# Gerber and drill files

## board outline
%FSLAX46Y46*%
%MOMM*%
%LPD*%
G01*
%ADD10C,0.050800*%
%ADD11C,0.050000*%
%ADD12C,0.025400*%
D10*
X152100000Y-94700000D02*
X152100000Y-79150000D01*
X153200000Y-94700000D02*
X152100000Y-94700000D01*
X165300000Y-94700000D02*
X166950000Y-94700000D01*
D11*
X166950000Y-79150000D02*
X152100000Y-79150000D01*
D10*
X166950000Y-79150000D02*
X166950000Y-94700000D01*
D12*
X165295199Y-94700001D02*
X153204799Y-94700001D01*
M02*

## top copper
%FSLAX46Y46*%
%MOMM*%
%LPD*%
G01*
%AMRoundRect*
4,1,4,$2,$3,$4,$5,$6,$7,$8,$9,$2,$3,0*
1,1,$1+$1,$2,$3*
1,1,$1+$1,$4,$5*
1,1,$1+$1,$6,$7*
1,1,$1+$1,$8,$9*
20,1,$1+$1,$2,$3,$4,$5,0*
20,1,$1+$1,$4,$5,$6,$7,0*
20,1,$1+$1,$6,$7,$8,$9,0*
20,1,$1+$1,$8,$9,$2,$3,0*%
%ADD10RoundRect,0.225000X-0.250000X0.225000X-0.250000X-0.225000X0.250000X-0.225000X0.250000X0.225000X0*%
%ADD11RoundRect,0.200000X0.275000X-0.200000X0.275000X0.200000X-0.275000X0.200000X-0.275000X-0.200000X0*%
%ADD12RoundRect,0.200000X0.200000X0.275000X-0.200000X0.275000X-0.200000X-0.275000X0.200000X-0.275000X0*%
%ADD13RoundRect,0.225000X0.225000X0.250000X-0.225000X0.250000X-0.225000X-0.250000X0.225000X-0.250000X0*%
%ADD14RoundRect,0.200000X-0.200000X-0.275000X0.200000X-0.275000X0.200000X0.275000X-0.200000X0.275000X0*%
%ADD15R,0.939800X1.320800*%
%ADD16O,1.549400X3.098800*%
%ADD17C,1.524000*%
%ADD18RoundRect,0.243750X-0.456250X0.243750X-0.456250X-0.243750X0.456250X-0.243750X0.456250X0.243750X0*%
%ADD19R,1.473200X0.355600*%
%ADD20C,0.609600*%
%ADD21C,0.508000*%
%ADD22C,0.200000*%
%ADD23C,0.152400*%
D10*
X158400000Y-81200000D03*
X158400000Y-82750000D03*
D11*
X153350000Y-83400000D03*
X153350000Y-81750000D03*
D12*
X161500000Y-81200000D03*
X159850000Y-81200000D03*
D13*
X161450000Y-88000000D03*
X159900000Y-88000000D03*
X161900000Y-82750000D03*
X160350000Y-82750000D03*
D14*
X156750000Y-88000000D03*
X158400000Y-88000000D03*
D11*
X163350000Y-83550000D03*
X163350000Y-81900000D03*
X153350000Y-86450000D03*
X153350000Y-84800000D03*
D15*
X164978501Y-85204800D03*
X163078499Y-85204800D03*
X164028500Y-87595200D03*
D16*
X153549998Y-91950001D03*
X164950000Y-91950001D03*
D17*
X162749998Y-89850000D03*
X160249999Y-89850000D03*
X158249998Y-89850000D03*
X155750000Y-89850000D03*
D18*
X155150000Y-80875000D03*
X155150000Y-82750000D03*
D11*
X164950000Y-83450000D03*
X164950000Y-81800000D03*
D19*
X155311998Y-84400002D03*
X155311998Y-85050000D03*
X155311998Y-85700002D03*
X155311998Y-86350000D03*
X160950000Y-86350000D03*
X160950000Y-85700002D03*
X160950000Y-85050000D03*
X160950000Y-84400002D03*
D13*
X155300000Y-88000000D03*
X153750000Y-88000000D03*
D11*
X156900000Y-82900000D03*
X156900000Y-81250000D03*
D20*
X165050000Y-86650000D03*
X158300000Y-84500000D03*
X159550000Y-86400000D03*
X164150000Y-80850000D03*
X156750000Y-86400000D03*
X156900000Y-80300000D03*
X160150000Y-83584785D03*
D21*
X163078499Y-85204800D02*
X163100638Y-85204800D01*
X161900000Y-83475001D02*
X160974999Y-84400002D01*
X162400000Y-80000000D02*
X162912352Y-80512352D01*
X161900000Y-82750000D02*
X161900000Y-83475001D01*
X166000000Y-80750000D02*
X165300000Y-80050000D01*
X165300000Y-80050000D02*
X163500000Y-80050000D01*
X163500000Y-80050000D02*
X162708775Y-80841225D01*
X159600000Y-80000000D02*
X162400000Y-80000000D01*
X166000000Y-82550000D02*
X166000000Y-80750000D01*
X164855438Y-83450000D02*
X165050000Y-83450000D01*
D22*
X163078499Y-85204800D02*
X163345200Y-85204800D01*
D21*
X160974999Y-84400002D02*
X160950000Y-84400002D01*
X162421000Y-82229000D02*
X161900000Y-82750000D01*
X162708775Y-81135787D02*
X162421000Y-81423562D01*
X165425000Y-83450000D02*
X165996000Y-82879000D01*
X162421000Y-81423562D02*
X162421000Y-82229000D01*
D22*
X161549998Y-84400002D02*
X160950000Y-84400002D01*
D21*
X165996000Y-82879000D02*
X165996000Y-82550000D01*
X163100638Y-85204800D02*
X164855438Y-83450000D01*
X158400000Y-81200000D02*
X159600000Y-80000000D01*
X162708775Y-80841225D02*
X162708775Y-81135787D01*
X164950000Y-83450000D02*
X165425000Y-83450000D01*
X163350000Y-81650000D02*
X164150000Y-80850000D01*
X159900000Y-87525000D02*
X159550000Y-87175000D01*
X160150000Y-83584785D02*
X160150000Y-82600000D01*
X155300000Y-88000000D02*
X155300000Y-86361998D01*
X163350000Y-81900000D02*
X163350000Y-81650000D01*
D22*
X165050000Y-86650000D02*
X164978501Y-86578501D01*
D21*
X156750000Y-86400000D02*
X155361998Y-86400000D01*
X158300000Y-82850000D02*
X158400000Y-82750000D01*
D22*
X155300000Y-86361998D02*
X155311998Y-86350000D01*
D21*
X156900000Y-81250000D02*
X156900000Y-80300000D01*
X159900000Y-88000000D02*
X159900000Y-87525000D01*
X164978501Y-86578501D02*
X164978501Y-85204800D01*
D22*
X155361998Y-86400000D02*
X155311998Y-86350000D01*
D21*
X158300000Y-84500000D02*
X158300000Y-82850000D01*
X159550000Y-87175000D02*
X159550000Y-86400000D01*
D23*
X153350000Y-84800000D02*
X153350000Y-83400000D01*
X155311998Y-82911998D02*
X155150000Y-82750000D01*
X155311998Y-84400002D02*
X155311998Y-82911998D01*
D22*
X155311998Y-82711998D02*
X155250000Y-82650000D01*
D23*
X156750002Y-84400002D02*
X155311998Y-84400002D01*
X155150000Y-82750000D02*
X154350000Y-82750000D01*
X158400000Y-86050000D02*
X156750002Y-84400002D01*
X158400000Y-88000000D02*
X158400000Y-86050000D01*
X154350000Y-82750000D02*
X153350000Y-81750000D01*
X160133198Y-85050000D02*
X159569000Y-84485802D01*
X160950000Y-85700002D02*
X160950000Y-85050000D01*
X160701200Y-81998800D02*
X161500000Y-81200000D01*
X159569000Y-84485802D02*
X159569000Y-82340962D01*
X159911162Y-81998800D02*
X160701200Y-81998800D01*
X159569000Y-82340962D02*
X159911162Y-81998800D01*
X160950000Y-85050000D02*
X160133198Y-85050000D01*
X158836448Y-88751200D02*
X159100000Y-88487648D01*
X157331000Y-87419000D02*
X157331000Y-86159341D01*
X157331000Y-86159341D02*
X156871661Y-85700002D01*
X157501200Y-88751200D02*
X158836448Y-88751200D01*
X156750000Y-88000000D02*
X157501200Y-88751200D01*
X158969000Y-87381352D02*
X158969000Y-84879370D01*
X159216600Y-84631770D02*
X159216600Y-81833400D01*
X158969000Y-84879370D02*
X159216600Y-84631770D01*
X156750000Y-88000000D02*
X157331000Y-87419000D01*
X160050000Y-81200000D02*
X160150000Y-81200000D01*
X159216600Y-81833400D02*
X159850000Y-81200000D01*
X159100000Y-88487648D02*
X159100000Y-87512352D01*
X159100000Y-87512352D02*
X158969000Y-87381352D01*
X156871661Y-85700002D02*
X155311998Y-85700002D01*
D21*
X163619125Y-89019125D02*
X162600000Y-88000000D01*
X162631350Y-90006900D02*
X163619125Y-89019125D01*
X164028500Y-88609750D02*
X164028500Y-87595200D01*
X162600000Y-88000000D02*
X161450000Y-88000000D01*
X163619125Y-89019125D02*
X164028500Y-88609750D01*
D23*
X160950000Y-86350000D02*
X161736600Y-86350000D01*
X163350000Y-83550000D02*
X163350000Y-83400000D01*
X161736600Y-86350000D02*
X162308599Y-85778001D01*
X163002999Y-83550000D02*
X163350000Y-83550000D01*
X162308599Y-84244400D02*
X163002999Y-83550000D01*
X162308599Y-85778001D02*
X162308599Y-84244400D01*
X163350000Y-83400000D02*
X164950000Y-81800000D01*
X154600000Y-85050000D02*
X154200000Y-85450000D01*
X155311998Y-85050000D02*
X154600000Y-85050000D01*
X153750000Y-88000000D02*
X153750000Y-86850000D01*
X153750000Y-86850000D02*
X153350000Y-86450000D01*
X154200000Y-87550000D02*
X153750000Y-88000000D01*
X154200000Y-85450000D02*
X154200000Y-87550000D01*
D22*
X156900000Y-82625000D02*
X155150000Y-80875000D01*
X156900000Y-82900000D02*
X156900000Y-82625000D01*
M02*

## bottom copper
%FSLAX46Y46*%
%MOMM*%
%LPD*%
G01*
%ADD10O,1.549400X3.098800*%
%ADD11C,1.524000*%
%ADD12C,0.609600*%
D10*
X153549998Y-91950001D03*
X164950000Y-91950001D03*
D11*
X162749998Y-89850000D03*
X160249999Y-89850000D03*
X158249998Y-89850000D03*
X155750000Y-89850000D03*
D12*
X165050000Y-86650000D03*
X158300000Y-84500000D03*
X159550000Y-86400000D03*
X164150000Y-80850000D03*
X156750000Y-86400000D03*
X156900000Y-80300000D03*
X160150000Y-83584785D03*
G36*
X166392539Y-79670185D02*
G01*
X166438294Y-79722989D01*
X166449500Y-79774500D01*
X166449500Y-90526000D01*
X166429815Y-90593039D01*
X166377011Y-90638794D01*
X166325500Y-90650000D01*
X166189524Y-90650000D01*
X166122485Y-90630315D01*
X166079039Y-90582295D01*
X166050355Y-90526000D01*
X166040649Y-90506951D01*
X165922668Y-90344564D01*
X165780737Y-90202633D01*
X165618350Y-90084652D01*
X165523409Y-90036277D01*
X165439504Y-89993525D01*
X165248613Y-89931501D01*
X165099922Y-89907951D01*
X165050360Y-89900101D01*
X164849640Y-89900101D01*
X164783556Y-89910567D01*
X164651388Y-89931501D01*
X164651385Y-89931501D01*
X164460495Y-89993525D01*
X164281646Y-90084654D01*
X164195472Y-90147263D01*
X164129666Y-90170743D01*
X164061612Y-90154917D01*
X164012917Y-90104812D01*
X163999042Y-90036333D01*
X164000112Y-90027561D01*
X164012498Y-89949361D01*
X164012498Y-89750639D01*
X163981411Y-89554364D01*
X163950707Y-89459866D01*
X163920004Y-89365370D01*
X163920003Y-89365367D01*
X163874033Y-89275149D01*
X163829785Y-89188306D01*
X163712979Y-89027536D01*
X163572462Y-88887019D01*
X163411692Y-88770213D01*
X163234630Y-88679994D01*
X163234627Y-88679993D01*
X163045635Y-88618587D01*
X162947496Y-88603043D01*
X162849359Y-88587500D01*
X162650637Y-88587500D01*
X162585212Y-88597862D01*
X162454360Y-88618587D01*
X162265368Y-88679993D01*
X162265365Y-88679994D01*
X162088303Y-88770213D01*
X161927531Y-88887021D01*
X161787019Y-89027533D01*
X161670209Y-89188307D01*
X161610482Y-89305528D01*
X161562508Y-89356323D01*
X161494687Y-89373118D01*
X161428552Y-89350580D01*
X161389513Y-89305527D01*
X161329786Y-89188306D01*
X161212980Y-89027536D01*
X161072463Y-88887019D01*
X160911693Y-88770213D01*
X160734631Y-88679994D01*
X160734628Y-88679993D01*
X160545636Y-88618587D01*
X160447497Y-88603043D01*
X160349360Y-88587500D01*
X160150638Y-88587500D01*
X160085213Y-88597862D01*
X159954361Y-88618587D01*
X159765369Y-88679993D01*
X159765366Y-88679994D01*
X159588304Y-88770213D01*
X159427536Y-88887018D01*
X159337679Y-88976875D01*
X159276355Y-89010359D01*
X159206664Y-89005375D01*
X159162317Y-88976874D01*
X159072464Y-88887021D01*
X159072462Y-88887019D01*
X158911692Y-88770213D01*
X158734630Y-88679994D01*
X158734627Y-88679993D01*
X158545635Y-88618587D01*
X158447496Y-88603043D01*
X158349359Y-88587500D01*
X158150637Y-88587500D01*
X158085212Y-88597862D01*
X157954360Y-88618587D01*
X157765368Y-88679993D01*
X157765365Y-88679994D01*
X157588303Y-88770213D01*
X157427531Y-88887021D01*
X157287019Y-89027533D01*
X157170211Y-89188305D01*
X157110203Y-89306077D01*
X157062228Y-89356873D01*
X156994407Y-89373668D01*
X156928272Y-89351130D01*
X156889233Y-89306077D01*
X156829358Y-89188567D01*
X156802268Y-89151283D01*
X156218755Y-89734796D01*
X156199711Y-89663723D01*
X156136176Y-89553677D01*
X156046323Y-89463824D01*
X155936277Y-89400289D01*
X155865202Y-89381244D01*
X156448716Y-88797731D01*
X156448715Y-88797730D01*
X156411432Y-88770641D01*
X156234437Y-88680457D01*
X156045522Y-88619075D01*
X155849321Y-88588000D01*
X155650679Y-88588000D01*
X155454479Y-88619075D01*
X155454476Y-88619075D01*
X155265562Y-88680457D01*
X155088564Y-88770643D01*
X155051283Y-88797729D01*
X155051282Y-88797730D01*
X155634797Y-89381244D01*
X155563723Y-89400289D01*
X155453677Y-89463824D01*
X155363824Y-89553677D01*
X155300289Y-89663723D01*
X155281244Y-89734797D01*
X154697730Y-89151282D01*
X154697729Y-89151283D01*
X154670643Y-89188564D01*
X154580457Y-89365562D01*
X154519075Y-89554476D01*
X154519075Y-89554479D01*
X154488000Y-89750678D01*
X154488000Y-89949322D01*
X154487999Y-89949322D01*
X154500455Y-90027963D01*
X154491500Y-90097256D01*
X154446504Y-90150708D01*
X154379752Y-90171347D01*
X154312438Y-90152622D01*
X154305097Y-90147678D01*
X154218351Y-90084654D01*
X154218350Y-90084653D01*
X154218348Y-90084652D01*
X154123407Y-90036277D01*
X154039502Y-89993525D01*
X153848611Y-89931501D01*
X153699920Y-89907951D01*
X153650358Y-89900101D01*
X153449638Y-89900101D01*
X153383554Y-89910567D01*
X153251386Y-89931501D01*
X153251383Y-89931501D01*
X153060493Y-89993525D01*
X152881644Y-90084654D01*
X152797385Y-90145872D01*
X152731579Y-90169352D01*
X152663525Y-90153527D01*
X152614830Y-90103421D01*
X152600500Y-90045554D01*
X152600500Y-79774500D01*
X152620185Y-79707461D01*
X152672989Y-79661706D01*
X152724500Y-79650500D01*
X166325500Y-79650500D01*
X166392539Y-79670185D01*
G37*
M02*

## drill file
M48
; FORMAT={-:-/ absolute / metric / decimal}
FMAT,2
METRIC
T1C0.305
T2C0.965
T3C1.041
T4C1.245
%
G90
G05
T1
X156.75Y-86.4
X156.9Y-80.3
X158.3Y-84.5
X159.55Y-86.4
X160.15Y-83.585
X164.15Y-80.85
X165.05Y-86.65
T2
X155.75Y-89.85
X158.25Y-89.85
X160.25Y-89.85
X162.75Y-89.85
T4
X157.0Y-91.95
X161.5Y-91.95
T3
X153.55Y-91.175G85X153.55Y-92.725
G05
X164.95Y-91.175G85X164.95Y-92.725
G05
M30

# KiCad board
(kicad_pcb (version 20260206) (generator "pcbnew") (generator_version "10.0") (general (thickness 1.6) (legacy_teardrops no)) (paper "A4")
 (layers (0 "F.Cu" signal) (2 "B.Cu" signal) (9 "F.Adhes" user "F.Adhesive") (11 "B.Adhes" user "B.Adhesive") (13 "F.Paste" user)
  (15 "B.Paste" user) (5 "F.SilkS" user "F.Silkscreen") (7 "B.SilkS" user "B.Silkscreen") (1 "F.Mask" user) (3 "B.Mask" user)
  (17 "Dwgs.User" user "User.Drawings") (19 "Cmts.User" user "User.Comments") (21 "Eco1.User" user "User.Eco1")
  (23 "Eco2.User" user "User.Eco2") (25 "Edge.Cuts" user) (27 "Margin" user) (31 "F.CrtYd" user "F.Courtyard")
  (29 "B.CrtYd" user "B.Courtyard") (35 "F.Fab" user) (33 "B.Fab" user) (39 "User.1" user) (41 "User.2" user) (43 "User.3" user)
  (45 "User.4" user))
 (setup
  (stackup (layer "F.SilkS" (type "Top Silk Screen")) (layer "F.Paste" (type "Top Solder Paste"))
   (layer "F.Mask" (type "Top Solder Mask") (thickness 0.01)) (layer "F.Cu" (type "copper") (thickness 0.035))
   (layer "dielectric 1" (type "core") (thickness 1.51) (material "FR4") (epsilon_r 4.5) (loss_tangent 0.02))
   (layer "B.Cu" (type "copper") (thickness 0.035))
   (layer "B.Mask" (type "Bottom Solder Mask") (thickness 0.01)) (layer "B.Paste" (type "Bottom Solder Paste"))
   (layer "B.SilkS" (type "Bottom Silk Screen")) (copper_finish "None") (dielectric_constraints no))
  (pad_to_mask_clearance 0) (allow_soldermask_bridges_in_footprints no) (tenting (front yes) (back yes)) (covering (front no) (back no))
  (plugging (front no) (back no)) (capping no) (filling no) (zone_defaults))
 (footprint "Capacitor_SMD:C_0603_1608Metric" (layer "F.Cu") (at 158.4 81.975 -90)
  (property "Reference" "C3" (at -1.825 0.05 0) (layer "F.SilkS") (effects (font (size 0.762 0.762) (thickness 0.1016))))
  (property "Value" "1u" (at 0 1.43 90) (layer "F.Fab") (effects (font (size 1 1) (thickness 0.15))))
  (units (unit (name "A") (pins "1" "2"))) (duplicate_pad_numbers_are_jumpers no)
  (pad "1" smd roundrect (at -0.775 0 270) (size 0.9 0.95) (layers "F.Cu" "F.Mask" "F.Paste") (roundrect_rratio 0.25) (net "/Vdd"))
  (pad "2" smd roundrect (at 0.775 0 270) (size 0.9 0.95) (layers "F.Cu" "F.Mask" "F.Paste") (roundrect_rratio 0.25) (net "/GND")))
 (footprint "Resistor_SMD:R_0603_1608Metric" (layer "F.Cu") (at 153.35 82.575 90)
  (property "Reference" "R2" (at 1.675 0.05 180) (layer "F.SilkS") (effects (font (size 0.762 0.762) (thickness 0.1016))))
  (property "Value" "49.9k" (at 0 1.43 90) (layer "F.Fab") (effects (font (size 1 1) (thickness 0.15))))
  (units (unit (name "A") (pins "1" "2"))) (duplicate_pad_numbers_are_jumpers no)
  (pad "1" smd roundrect (at -0.825 0 90) (size 0.8 0.95) (layers "F.Cu" "F.Mask" "F.Paste") (roundrect_rratio 0.25) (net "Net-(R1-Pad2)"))
  (pad "2" smd roundrect (at 0.825 0 90) (size 0.8 0.95) (layers "F.Cu" "F.Mask" "F.Paste") (roundrect_rratio 0.25) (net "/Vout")))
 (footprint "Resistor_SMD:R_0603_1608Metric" (layer "F.Cu") (at 160.675 81.2 180)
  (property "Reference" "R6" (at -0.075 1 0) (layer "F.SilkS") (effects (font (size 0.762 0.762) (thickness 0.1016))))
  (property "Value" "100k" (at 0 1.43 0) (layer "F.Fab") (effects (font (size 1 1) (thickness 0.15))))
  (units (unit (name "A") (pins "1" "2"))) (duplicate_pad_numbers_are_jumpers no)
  (pad "1" smd roundrect (at -0.825 0 180) (size 0.8 0.95) (layers "F.Cu" "F.Mask" "F.Paste") (roundrect_rratio 0.25) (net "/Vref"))
  (pad "2" smd roundrect (at 0.825 0 180) (size 0.8 0.95) (layers "F.Cu" "F.Mask" "F.Paste") (roundrect_rratio 0.25) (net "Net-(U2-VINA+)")))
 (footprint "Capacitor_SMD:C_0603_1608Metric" (layer "F.Cu") (at 160.675 88 180)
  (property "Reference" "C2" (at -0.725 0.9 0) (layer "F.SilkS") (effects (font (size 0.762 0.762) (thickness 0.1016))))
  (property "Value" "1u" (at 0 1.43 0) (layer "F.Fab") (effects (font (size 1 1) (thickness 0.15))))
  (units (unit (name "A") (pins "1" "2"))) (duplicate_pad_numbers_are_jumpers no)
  (pad "1" smd roundrect (at -0.775 0 180) (size 0.9 0.95) (layers "F.Cu" "F.Mask" "F.Paste") (roundrect_rratio 0.25) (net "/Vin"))
  (pad "2" smd roundrect (at 0.775 0 180) (size 0.9 0.95) (layers "F.Cu" "F.Mask" "F.Paste") (roundrect_rratio 0.25) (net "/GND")))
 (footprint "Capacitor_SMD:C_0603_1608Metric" (layer "F.Cu") (at 161.125 82.75 180)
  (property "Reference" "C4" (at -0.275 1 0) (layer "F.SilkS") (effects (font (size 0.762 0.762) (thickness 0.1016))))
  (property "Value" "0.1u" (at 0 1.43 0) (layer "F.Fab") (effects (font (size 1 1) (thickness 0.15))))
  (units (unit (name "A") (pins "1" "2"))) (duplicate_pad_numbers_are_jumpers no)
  (pad "1" smd roundrect (at -0.775 0 180) (size 0.9 0.95) (layers "F.Cu" "F.Mask" "F.Paste") (roundrect_rratio 0.25) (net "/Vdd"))
  (pad "2" smd roundrect (at 0.775 0 180) (size 0.9 0.95) (layers "F.Cu" "F.Mask" "F.Paste") (roundrect_rratio 0.25) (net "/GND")))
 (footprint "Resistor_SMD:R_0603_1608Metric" (layer "F.Cu") (at 157.575 88)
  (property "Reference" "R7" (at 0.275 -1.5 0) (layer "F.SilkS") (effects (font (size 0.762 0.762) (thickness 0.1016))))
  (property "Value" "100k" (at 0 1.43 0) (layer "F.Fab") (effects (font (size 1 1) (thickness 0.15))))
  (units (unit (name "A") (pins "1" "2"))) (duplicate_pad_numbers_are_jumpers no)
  (pad "1" smd roundrect (at -0.825 0) (size 0.8 0.95) (layers "F.Cu" "F.Mask" "F.Paste") (roundrect_rratio 0.25) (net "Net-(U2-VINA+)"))
  (pad "2" smd roundrect (at 0.825 0) (size 0.8 0.95) (layers "F.Cu" "F.Mask" "F.Paste") (roundrect_rratio 0.25) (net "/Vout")))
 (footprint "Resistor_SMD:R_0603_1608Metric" (layer "F.Cu") (at 163.35 82.725 90)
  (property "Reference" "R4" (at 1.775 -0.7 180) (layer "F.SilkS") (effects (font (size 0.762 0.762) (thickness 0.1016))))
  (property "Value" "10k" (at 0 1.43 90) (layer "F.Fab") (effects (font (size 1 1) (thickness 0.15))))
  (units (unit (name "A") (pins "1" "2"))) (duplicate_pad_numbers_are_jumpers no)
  (pad "1" smd roundrect (at -0.825 0 90) (size 0.8 0.95) (layers "F.Cu" "F.Mask" "F.Paste") (roundrect_rratio 0.25) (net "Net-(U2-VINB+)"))
  (pad "2" smd roundrect (at 0.825 0 90) (size 0.8 0.95) (layers "F.Cu" "F.Mask" "F.Paste") (roundrect_rratio 0.25) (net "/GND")))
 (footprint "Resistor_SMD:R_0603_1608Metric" (layer "F.Cu") (at 153.35 85.625 90)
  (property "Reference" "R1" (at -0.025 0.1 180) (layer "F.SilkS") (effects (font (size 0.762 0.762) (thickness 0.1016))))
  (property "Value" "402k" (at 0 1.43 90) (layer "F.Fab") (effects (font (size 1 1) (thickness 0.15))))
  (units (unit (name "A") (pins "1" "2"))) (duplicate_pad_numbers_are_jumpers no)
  (pad "1" smd roundrect (at -0.825 0 90) (size 0.8 0.95) (layers "F.Cu" "F.Mask" "F.Paste") (roundrect_rratio 0.25) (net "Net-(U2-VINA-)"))
  (pad "2" smd roundrect (at 0.825 0 90) (size 0.8 0.95) (layers "F.Cu" "F.Mask" "F.Paste") (roundrect_rratio 0.25) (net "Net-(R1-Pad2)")))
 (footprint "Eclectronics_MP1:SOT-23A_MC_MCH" (layer "F.Cu") (at 164.0285 86.4 180)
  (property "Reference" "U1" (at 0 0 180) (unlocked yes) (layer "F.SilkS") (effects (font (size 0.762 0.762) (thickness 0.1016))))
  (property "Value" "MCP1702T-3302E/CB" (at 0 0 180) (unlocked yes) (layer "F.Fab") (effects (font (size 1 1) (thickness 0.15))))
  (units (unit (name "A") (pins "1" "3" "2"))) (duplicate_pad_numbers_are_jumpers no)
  (pad "1" smd rect (at -0.950001 1.1952 180) (size 0.9398 1.3208) (layers "F.Cu" "F.Mask" "F.Paste") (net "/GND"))
  (pad "2" smd rect (at 0.950001 1.1952 180) (size 0.9398 1.3208) (layers "F.Cu" "F.Mask" "F.Paste") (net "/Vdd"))
  (pad "3" smd rect (at 0 -1.1952 180) (size 0.9398 1.3208) (layers "F.Cu" "F.Mask" "F.Paste") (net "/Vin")))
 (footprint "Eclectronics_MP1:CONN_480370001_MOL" (layer "F.Cu") (at 162.749998 89.85)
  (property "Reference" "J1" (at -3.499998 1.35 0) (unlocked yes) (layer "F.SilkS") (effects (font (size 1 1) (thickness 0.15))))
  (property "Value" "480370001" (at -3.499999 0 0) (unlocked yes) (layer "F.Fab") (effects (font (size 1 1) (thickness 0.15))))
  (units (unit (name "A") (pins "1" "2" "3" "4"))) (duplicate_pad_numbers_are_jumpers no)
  (fp_line (start 2.545201 4.850001) (end -9.545199 4.850001) (stroke (width 0.0254) (type solid)) (layer "Edge.Cuts"))
  (pad "" np_thru_hole oval (at -9.2 2.100001) (size 1.5494 3.0988) (drill oval 1.0414 2.5908) (layers "*.Cu" "*.Mask"))
  (pad "" np_thru_hole circle (at -5.75 2.100001) (size 1.2446 1.2446) (drill 1.2446) (layers))
  (pad "" np_thru_hole circle (at -1.249999 2.100001) (size 1.2446 1.2446) (drill 1.2446) (layers))
  (pad "" np_thru_hole oval (at 2.200002 2.100001) (size 1.5494 3.0988) (drill oval 1.0414 2.5908) (layers "*.Cu" "*.Mask"))
  (pad "1" thru_hole circle (at 0 0) (size 1.524 1.524) (drill 0.9652) (layers "*.Cu" "*.Mask") (remove_unused_layers no) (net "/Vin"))
  (pad "2" thru_hole circle (at -2.499999 0) (size 1.524 1.524) (drill 0.9652) (layers "*.Cu" "*.Mask") (remove_unused_layers no)
   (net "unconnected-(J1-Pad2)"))
  (pad "3" thru_hole circle (at -4.5 0) (size 1.524 1.524) (drill 0.9652) (layers "*.Cu" "*.Mask") (remove_unused_layers no)
   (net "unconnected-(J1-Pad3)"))
  (pad "4" thru_hole circle (at -6.999998 0) (size 1.524 1.524) (drill 0.9652) (layers "*.Cu" "*.Mask") (remove_unused_layers no)
   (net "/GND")))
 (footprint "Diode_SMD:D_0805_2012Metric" (layer "F.Cu") (at 155.15 81.8125 -90)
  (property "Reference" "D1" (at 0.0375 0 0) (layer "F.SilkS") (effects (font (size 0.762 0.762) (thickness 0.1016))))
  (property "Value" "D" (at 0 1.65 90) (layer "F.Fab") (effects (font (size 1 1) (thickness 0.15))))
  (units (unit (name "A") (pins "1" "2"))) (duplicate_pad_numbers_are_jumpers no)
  (pad "1" smd roundrect (at -0.9375 0 270) (size 0.975 1.4) (layers "F.Cu" "F.Mask" "F.Paste") (roundrect_rratio 0.25) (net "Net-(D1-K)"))
  (pad "2" smd roundrect (at 0.9375 0 270) (size 0.975 1.4) (layers "F.Cu" "F.Mask" "F.Paste") (roundrect_rratio 0.25) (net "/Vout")))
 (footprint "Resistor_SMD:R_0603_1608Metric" (layer "F.Cu") (at 164.95 82.625 90)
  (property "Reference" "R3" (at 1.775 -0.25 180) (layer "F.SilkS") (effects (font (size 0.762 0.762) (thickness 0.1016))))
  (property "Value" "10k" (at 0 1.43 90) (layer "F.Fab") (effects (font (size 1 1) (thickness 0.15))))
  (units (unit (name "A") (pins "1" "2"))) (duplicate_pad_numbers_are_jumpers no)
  (pad "1" smd roundrect (at -0.825 0 90) (size 0.8 0.95) (layers "F.Cu" "F.Mask" "F.Paste") (roundrect_rratio 0.25) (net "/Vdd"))
  (pad "2" smd roundrect (at 0.825 0 90) (size 0.8 0.95) (layers "F.Cu" "F.Mask" "F.Paste") (roundrect_rratio 0.25) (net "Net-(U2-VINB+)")))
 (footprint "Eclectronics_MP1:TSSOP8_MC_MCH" (layer "F.Cu") (at 158.130999 85.375001)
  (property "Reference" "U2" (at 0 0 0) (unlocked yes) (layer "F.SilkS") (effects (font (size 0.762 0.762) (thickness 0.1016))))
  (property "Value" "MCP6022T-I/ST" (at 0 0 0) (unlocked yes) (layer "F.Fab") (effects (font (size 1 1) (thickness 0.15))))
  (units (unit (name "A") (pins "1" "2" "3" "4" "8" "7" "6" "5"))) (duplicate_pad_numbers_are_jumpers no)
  (pad "1" smd rect (at -2.819001 -0.974999) (size 1.4732 0.3556) (layers "F.Cu" "F.Mask" "F.Paste") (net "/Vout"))
  (pad "2" smd rect (at -2.819001 -0.325001) (size 1.4732 0.3556) (layers "F.Cu" "F.Mask" "F.Paste") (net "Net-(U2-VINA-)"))
  (pad "3" smd rect (at -2.819001 0.325001) (size 1.4732 0.3556) (layers "F.Cu" "F.Mask" "F.Paste") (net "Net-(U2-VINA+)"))
  (pad "4" smd rect (at -2.819001 0.974999) (size 1.4732 0.3556) (layers "F.Cu" "F.Mask" "F.Paste") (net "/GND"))
  (pad "5" smd rect (at 2.819001 0.974999) (size 1.4732 0.3556) (layers "F.Cu" "F.Mask" "F.Paste") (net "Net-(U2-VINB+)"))
  (pad "6" smd rect (at 2.819001 0.325001) (size 1.4732 0.3556) (layers "F.Cu" "F.Mask" "F.Paste") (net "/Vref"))
  (pad "7" smd rect (at 2.819001 -0.325001) (size 1.4732 0.3556) (layers "F.Cu" "F.Mask" "F.Paste") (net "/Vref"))
  (pad "8" smd rect (at 2.819001 -0.974999) (size 1.4732 0.3556) (layers "F.Cu" "F.Mask" "F.Paste") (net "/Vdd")))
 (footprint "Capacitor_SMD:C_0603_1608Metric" (layer "F.Cu") (at 154.525 88 180)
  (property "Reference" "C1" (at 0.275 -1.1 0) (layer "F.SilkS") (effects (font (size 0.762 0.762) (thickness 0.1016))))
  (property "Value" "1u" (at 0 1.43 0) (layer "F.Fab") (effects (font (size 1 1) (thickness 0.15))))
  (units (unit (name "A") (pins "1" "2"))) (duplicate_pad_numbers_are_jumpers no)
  (pad "1" smd roundrect (at -0.775 0 180) (size 0.9 0.95) (layers "F.Cu" "F.Mask" "F.Paste") (roundrect_rratio 0.25) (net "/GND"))
  (pad "2" smd roundrect (at 0.775 0 180) (size 0.9 0.95) (layers "F.Cu" "F.Mask" "F.Paste") (roundrect_rratio 0.25) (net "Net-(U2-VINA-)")))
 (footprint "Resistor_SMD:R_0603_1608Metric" (layer "F.Cu") (at 156.9 82.075 90)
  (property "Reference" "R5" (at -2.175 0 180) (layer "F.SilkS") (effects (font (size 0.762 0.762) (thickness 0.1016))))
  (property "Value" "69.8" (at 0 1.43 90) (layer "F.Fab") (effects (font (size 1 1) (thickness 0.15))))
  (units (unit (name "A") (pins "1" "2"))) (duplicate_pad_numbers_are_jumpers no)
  (pad "1" smd roundrect (at -0.825 0 90) (size 0.8 0.95) (layers "F.Cu" "F.Mask" "F.Paste") (roundrect_rratio 0.25) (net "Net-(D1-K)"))
  (pad "2" smd roundrect (at 0.825 0 90) (size 0.8 0.95) (layers "F.Cu" "F.Mask" "F.Paste") (roundrect_rratio 0.25) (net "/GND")))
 (gr_line (start 152.1 94.7) (end 152.1 79.15) (stroke (width 0.0508) (type solid)) (layer "Edge.Cuts"))
 (gr_line (start 153.2 94.7) (end 152.1 94.7) (stroke (width 0.0508) (type solid)) (layer "Edge.Cuts"))
 (gr_line (start 165.3 94.7) (end 166.95 94.7) (stroke (width 0.0508) (type solid)) (layer "Edge.Cuts"))
 (gr_line (start 166.95 79.15) (end 152.1 79.15) (stroke (width 0.05) (type default)) (layer "Edge.Cuts"))
 (gr_line (start 166.95 79.15) (end 166.95 94.7) (stroke (width 0.0508) (type solid)) (layer "Edge.Cuts"))
 (segment (start 163.078499 85.2048) (end 163.100638 85.2048) (width 0.508) (layer "F.Cu") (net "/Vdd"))
 (segment (start 161.9 83.475001) (end 160.974999 84.400002) (width 0.508) (layer "F.Cu") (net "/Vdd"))
 (segment (start 162.4 80) (end 162.912352 80.512352) (width 0.508) (layer "F.Cu") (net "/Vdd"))
 (segment (start 161.9 82.75) (end 161.9 83.475001) (width 0.508) (layer "F.Cu") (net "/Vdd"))
 (segment (start 166 80.75) (end 165.3 80.05) (width 0.508) (layer "F.Cu") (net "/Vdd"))
 (segment (start 165.3 80.05) (end 163.5 80.05) (width 0.508) (layer "F.Cu") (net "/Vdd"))
 (segment (start 163.5 80.05) (end 162.708775 80.841225) (width 0.508) (layer "F.Cu") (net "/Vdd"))
 (segment (start 159.6 80) (end 162.4 80) (width 0.508) (layer "F.Cu") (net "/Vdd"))
 (segment (start 166 82.55) (end 166 80.75) (width 0.508) (layer "F.Cu") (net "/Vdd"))
 (segment (start 164.855438 83.45) (end 165.05 83.45) (width 0.508) (layer "F.Cu") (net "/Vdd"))
 (segment (start 163.078499 85.2048) (end 163.3452 85.2048) (width 0.2) (layer "F.Cu") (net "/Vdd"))
 (segment (start 160.974999 84.400002) (end 160.95 84.400002) (width 0.508) (layer "F.Cu") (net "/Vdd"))
 (segment (start 162.421 82.229) (end 161.9 82.75) (width 0.508) (layer "F.Cu") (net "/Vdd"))
 (segment (start 162.708775 81.135787) (end 162.421 81.423562) (width 0.508) (layer "F.Cu") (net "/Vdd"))
 (segment (start 165.425 83.45) (end 165.996 82.879) (width 0.508) (layer "F.Cu") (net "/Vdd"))
 (segment (start 162.421 81.423562) (end 162.421 82.229) (width 0.508) (layer "F.Cu") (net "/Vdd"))
 (segment (start 161.549998 84.400002) (end 160.95 84.400002) (width 0.2) (layer "F.Cu") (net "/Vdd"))
 (segment (start 165.996 82.879) (end 165.996 82.55) (width 0.508) (layer "F.Cu") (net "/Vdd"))
 (segment (start 163.100638 85.2048) (end 164.855438 83.45) (width 0.508) (layer "F.Cu") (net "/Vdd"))
 (segment (start 158.4 81.2) (end 159.6 80) (width 0.508) (layer "F.Cu") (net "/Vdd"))
 (segment (start 162.708775 80.841225) (end 162.708775 81.135787) (width 0.508) (layer "F.Cu") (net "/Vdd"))
 (segment (start 164.95 83.45) (end 165.425 83.45) (width 0.508) (layer "F.Cu") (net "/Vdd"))
 (segment (start 163.35 81.65) (end 164.15 80.85) (width 0.508) (layer "F.Cu") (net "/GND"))
 (segment (start 159.9 87.525) (end 159.55 87.175) (width 0.508) (layer "F.Cu") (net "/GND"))
 (segment (start 160.15 83.584785) (end 160.15 82.6) (width 0.508) (layer "F.Cu") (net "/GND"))
 (segment (start 155.3 88) (end 155.3 86.361998) (width 0.508) (layer "F.Cu") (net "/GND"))
 (segment (start 163.35 81.9) (end 163.35 81.65) (width 0.508) (layer "F.Cu") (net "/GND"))
 (segment (start 165.05 86.65) (end 164.978501 86.578501) (width 0.2) (layer "F.Cu") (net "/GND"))
 (segment (start 156.75 86.4) (end 155.361998 86.4) (width 0.508) (layer "F.Cu") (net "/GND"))
 (segment (start 158.3 82.85) (end 158.4 82.75) (width 0.508) (layer "F.Cu") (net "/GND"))
 (segment (start 155.3 86.361998) (end 155.311998 86.35) (width 0.2) (layer "F.Cu") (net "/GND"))
 (segment (start 156.9 81.25) (end 156.9 80.3) (width 0.508) (layer "F.Cu") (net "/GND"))
 (segment (start 159.9 88) (end 159.9 87.525) (width 0.508) (layer "F.Cu") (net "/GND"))
 (segment (start 164.978501 86.578501) (end 164.978501 85.2048) (width 0.508) (layer "F.Cu") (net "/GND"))
 (segment (start 155.361998 86.4) (end 155.311998 86.35) (width 0.2) (layer "F.Cu") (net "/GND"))
 (segment (start 158.3 84.5) (end 158.3 82.85) (width 0.508) (layer "F.Cu") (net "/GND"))
 (segment (start 159.55 87.175) (end 159.55 86.4) (width 0.508) (layer "F.Cu") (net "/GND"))
 (via (at 165.05 86.65) (size 0.6096) (drill 0.3048) (layers "F.Cu" "B.Cu") (free yes) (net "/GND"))
 (via (at 158.3 84.5) (size 0.6096) (drill 0.3048) (layers "F.Cu" "B.Cu") (free yes) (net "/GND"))
 (via (at 159.55 86.4) (size 0.6096) (drill 0.3048) (layers "F.Cu" "B.Cu") (free yes) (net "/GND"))
 (via (at 164.15 80.85) (size 0.6096) (drill 0.3048) (layers "F.Cu" "B.Cu") (free yes) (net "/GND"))
 (via (at 156.75 86.4) (size 0.6096) (drill 0.3048) (layers "F.Cu" "B.Cu") (free yes) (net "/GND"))
 (via (at 156.9 80.3) (size 0.6096) (drill 0.3048) (layers "F.Cu" "B.Cu") (free yes) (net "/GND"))
 (via (at 160.15 83.584785) (size 0.6096) (drill 0.3048) (layers "F.Cu" "B.Cu") (free yes) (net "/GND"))
 (segment (start 153.35 84.8) (end 153.35 83.4) (width 0.1524) (layer "F.Cu") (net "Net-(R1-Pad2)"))
 (segment (start 155.311998 82.911998) (end 155.15 82.75) (width 0.1524) (layer "F.Cu") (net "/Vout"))
 (segment (start 155.311998 84.400002) (end 155.311998 82.911998) (width 0.1524) (layer "F.Cu") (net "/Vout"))
 (segment (start 155.311998 82.711998) (end 155.25 82.65) (width 0.2) (layer "F.Cu") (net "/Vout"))
 (segment (start 156.750002 84.400002) (end 155.311998 84.400002) (width 0.1524) (layer "F.Cu") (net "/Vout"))
 (segment (start 155.15 82.75) (end 154.35 82.75) (width 0.1524) (layer "F.Cu") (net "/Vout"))
 (segment (start 158.4 86.05) (end 156.750002 84.400002) (width 0.1524) (layer "F.Cu") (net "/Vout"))
 (segment (start 158.4 88) (end 158.4 86.05) (width 0.1524) (layer "F.Cu") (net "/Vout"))
 (segment (start 154.35 82.75) (end 153.35 81.75) (width 0.1524) (layer "F.Cu") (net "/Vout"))
 (segment (start 160.133198 85.05) (end 159.569 84.485802) (width 0.1524) (layer "F.Cu") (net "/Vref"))
 (segment (start 160.95 85.700002) (end 160.95 85.05) (width 0.1524) (layer "F.Cu") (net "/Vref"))
 (segment (start 160.7012 81.9988) (end 161.5 81.2) (width 0.1524) (layer "F.Cu") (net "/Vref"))
 (segment (start 159.569 84.485802) (end 159.569 82.340962) (width 0.1524) (layer "F.Cu") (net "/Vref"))
 (segment (start 159.911162 81.9988) (end 160.7012 81.9988) (width 0.1524) (layer "F.Cu") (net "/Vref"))
 (segment (start 159.569 82.340962) (end 159.911162 81.9988) (width 0.1524) (layer "F.Cu") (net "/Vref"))
 (segment (start 160.95 85.05) (end 160.133198 85.05) (width 0.1524) (layer "F.Cu") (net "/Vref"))
 (segment (start 158.836448 88.7512) (end 159.1 88.487648) (width 0.1524) (layer "F.Cu") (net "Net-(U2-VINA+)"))
 (segment (start 157.331 87.419) (end 157.331 86.159341) (width 0.1524) (layer "F.Cu") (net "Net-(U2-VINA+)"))
 (segment (start 157.331 86.159341) (end 156.871661 85.700002) (width 0.1524) (layer "F.Cu") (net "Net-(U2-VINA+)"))
 (segment (start 157.5012 88.7512) (end 158.836448 88.7512) (width 0.1524) (layer "F.Cu") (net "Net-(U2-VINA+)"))
 (segment (start 156.75 88) (end 157.5012 88.7512) (width 0.1524) (layer "F.Cu") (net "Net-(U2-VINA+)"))
 (segment (start 158.969 87.381352) (end 158.969 84.87937) (width 0.1524) (layer "F.Cu") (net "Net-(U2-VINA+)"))
 (segment (start 159.2166 84.63177) (end 159.2166 81.8334) (width 0.1524) (layer "F.Cu") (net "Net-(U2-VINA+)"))
 (segment (start 158.969 84.87937) (end 159.2166 84.63177) (width 0.1524) (layer "F.Cu") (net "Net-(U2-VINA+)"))
 (segment (start 156.75 88) (end 157.331 87.419) (width 0.1524) (layer "F.Cu") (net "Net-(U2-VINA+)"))
 (segment (start 160.05 81.2) (end 160.15 81.2) (width 0.1524) (layer "F.Cu") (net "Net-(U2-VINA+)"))
 (segment (start 159.2166 81.8334) (end 159.85 81.2) (width 0.1524) (layer "F.Cu") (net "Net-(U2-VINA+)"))
 (segment (start 159.1 88.487648) (end 159.1 87.512352) (width 0.1524) (layer "F.Cu") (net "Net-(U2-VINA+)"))
 (segment (start 159.1 87.512352) (end 158.969 87.381352) (width 0.1524) (layer "F.Cu") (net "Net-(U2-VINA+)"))
 (segment (start 156.871661 85.700002) (end 155.311998 85.700002) (width 0.1524) (layer "F.Cu") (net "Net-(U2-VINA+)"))
 (segment (start 163.619125 89.019125) (end 162.6 88) (width 0.508) (layer "F.Cu") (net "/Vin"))
 (segment (start 162.63135 90.0069) (end 163.619125 89.019125) (width 0.508) (layer "F.Cu") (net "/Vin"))
 (segment (start 164.0285 88.60975) (end 164.0285 87.5952) (width 0.508) (layer "F.Cu") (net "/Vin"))
 (segment (start 162.6 88) (end 161.45 88) (width 0.508) (layer "F.Cu") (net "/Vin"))
 (segment (start 163.619125 89.019125) (end 164.0285 88.60975) (width 0.508) (layer "F.Cu") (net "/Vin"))
 (segment (start 160.95 86.35) (end 161.7366 86.35) (width 0.1524) (layer "F.Cu") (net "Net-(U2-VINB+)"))
 (segment (start 163.35 83.55) (end 163.35 83.4) (width 0.1524) (layer "F.Cu") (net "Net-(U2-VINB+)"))
 (segment (start 161.7366 86.35) (end 162.308599 85.778001) (width 0.1524) (layer "F.Cu") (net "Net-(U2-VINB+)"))
 (segment (start 163.002999 83.55) (end 163.35 83.55) (width 0.1524) (layer "F.Cu") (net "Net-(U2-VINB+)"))
 (segment (start 162.308599 84.2444) (end 163.002999 83.55) (width 0.1524) (layer "F.Cu") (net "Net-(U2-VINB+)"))
 (segment (start 162.308599 85.778001) (end 162.308599 84.2444) (width 0.1524) (layer "F.Cu") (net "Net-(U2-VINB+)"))
 (segment (start 163.35 83.4) (end 164.95 81.8) (width 0.1524) (layer "F.Cu") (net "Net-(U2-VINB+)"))
 (segment (start 154.6 85.05) (end 154.2 85.45) (width 0.1524) (layer "F.Cu") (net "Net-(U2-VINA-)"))
 (segment (start 155.311998 85.05) (end 154.6 85.05) (width 0.1524) (layer "F.Cu") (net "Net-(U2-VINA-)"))
 (segment (start 153.75 88) (end 153.75 86.85) (width 0.1524) (layer "F.Cu") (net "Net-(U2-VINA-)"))
 (segment (start 153.75 86.85) (end 153.35 86.45) (width 0.1524) (layer "F.Cu") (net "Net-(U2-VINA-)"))
 (segment (start 154.2 87.55) (end 153.75 88) (width 0.1524) (layer "F.Cu") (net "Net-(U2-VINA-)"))
 (segment (start 154.2 85.45) (end 154.2 87.55) (width 0.1524) (layer "F.Cu") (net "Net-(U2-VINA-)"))
 (segment (start 156.9 82.625) (end 155.15 80.875) (width 0.2) (layer "F.Cu") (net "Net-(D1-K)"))
 (segment (start 156.9 82.9) (end 156.9 82.625) (width 0.2) (layer "F.Cu") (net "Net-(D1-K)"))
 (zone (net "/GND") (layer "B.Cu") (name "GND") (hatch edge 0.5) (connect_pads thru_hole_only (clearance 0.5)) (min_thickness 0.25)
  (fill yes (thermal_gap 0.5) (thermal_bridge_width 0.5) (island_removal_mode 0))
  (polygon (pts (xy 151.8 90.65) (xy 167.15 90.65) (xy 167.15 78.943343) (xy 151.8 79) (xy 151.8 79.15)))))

